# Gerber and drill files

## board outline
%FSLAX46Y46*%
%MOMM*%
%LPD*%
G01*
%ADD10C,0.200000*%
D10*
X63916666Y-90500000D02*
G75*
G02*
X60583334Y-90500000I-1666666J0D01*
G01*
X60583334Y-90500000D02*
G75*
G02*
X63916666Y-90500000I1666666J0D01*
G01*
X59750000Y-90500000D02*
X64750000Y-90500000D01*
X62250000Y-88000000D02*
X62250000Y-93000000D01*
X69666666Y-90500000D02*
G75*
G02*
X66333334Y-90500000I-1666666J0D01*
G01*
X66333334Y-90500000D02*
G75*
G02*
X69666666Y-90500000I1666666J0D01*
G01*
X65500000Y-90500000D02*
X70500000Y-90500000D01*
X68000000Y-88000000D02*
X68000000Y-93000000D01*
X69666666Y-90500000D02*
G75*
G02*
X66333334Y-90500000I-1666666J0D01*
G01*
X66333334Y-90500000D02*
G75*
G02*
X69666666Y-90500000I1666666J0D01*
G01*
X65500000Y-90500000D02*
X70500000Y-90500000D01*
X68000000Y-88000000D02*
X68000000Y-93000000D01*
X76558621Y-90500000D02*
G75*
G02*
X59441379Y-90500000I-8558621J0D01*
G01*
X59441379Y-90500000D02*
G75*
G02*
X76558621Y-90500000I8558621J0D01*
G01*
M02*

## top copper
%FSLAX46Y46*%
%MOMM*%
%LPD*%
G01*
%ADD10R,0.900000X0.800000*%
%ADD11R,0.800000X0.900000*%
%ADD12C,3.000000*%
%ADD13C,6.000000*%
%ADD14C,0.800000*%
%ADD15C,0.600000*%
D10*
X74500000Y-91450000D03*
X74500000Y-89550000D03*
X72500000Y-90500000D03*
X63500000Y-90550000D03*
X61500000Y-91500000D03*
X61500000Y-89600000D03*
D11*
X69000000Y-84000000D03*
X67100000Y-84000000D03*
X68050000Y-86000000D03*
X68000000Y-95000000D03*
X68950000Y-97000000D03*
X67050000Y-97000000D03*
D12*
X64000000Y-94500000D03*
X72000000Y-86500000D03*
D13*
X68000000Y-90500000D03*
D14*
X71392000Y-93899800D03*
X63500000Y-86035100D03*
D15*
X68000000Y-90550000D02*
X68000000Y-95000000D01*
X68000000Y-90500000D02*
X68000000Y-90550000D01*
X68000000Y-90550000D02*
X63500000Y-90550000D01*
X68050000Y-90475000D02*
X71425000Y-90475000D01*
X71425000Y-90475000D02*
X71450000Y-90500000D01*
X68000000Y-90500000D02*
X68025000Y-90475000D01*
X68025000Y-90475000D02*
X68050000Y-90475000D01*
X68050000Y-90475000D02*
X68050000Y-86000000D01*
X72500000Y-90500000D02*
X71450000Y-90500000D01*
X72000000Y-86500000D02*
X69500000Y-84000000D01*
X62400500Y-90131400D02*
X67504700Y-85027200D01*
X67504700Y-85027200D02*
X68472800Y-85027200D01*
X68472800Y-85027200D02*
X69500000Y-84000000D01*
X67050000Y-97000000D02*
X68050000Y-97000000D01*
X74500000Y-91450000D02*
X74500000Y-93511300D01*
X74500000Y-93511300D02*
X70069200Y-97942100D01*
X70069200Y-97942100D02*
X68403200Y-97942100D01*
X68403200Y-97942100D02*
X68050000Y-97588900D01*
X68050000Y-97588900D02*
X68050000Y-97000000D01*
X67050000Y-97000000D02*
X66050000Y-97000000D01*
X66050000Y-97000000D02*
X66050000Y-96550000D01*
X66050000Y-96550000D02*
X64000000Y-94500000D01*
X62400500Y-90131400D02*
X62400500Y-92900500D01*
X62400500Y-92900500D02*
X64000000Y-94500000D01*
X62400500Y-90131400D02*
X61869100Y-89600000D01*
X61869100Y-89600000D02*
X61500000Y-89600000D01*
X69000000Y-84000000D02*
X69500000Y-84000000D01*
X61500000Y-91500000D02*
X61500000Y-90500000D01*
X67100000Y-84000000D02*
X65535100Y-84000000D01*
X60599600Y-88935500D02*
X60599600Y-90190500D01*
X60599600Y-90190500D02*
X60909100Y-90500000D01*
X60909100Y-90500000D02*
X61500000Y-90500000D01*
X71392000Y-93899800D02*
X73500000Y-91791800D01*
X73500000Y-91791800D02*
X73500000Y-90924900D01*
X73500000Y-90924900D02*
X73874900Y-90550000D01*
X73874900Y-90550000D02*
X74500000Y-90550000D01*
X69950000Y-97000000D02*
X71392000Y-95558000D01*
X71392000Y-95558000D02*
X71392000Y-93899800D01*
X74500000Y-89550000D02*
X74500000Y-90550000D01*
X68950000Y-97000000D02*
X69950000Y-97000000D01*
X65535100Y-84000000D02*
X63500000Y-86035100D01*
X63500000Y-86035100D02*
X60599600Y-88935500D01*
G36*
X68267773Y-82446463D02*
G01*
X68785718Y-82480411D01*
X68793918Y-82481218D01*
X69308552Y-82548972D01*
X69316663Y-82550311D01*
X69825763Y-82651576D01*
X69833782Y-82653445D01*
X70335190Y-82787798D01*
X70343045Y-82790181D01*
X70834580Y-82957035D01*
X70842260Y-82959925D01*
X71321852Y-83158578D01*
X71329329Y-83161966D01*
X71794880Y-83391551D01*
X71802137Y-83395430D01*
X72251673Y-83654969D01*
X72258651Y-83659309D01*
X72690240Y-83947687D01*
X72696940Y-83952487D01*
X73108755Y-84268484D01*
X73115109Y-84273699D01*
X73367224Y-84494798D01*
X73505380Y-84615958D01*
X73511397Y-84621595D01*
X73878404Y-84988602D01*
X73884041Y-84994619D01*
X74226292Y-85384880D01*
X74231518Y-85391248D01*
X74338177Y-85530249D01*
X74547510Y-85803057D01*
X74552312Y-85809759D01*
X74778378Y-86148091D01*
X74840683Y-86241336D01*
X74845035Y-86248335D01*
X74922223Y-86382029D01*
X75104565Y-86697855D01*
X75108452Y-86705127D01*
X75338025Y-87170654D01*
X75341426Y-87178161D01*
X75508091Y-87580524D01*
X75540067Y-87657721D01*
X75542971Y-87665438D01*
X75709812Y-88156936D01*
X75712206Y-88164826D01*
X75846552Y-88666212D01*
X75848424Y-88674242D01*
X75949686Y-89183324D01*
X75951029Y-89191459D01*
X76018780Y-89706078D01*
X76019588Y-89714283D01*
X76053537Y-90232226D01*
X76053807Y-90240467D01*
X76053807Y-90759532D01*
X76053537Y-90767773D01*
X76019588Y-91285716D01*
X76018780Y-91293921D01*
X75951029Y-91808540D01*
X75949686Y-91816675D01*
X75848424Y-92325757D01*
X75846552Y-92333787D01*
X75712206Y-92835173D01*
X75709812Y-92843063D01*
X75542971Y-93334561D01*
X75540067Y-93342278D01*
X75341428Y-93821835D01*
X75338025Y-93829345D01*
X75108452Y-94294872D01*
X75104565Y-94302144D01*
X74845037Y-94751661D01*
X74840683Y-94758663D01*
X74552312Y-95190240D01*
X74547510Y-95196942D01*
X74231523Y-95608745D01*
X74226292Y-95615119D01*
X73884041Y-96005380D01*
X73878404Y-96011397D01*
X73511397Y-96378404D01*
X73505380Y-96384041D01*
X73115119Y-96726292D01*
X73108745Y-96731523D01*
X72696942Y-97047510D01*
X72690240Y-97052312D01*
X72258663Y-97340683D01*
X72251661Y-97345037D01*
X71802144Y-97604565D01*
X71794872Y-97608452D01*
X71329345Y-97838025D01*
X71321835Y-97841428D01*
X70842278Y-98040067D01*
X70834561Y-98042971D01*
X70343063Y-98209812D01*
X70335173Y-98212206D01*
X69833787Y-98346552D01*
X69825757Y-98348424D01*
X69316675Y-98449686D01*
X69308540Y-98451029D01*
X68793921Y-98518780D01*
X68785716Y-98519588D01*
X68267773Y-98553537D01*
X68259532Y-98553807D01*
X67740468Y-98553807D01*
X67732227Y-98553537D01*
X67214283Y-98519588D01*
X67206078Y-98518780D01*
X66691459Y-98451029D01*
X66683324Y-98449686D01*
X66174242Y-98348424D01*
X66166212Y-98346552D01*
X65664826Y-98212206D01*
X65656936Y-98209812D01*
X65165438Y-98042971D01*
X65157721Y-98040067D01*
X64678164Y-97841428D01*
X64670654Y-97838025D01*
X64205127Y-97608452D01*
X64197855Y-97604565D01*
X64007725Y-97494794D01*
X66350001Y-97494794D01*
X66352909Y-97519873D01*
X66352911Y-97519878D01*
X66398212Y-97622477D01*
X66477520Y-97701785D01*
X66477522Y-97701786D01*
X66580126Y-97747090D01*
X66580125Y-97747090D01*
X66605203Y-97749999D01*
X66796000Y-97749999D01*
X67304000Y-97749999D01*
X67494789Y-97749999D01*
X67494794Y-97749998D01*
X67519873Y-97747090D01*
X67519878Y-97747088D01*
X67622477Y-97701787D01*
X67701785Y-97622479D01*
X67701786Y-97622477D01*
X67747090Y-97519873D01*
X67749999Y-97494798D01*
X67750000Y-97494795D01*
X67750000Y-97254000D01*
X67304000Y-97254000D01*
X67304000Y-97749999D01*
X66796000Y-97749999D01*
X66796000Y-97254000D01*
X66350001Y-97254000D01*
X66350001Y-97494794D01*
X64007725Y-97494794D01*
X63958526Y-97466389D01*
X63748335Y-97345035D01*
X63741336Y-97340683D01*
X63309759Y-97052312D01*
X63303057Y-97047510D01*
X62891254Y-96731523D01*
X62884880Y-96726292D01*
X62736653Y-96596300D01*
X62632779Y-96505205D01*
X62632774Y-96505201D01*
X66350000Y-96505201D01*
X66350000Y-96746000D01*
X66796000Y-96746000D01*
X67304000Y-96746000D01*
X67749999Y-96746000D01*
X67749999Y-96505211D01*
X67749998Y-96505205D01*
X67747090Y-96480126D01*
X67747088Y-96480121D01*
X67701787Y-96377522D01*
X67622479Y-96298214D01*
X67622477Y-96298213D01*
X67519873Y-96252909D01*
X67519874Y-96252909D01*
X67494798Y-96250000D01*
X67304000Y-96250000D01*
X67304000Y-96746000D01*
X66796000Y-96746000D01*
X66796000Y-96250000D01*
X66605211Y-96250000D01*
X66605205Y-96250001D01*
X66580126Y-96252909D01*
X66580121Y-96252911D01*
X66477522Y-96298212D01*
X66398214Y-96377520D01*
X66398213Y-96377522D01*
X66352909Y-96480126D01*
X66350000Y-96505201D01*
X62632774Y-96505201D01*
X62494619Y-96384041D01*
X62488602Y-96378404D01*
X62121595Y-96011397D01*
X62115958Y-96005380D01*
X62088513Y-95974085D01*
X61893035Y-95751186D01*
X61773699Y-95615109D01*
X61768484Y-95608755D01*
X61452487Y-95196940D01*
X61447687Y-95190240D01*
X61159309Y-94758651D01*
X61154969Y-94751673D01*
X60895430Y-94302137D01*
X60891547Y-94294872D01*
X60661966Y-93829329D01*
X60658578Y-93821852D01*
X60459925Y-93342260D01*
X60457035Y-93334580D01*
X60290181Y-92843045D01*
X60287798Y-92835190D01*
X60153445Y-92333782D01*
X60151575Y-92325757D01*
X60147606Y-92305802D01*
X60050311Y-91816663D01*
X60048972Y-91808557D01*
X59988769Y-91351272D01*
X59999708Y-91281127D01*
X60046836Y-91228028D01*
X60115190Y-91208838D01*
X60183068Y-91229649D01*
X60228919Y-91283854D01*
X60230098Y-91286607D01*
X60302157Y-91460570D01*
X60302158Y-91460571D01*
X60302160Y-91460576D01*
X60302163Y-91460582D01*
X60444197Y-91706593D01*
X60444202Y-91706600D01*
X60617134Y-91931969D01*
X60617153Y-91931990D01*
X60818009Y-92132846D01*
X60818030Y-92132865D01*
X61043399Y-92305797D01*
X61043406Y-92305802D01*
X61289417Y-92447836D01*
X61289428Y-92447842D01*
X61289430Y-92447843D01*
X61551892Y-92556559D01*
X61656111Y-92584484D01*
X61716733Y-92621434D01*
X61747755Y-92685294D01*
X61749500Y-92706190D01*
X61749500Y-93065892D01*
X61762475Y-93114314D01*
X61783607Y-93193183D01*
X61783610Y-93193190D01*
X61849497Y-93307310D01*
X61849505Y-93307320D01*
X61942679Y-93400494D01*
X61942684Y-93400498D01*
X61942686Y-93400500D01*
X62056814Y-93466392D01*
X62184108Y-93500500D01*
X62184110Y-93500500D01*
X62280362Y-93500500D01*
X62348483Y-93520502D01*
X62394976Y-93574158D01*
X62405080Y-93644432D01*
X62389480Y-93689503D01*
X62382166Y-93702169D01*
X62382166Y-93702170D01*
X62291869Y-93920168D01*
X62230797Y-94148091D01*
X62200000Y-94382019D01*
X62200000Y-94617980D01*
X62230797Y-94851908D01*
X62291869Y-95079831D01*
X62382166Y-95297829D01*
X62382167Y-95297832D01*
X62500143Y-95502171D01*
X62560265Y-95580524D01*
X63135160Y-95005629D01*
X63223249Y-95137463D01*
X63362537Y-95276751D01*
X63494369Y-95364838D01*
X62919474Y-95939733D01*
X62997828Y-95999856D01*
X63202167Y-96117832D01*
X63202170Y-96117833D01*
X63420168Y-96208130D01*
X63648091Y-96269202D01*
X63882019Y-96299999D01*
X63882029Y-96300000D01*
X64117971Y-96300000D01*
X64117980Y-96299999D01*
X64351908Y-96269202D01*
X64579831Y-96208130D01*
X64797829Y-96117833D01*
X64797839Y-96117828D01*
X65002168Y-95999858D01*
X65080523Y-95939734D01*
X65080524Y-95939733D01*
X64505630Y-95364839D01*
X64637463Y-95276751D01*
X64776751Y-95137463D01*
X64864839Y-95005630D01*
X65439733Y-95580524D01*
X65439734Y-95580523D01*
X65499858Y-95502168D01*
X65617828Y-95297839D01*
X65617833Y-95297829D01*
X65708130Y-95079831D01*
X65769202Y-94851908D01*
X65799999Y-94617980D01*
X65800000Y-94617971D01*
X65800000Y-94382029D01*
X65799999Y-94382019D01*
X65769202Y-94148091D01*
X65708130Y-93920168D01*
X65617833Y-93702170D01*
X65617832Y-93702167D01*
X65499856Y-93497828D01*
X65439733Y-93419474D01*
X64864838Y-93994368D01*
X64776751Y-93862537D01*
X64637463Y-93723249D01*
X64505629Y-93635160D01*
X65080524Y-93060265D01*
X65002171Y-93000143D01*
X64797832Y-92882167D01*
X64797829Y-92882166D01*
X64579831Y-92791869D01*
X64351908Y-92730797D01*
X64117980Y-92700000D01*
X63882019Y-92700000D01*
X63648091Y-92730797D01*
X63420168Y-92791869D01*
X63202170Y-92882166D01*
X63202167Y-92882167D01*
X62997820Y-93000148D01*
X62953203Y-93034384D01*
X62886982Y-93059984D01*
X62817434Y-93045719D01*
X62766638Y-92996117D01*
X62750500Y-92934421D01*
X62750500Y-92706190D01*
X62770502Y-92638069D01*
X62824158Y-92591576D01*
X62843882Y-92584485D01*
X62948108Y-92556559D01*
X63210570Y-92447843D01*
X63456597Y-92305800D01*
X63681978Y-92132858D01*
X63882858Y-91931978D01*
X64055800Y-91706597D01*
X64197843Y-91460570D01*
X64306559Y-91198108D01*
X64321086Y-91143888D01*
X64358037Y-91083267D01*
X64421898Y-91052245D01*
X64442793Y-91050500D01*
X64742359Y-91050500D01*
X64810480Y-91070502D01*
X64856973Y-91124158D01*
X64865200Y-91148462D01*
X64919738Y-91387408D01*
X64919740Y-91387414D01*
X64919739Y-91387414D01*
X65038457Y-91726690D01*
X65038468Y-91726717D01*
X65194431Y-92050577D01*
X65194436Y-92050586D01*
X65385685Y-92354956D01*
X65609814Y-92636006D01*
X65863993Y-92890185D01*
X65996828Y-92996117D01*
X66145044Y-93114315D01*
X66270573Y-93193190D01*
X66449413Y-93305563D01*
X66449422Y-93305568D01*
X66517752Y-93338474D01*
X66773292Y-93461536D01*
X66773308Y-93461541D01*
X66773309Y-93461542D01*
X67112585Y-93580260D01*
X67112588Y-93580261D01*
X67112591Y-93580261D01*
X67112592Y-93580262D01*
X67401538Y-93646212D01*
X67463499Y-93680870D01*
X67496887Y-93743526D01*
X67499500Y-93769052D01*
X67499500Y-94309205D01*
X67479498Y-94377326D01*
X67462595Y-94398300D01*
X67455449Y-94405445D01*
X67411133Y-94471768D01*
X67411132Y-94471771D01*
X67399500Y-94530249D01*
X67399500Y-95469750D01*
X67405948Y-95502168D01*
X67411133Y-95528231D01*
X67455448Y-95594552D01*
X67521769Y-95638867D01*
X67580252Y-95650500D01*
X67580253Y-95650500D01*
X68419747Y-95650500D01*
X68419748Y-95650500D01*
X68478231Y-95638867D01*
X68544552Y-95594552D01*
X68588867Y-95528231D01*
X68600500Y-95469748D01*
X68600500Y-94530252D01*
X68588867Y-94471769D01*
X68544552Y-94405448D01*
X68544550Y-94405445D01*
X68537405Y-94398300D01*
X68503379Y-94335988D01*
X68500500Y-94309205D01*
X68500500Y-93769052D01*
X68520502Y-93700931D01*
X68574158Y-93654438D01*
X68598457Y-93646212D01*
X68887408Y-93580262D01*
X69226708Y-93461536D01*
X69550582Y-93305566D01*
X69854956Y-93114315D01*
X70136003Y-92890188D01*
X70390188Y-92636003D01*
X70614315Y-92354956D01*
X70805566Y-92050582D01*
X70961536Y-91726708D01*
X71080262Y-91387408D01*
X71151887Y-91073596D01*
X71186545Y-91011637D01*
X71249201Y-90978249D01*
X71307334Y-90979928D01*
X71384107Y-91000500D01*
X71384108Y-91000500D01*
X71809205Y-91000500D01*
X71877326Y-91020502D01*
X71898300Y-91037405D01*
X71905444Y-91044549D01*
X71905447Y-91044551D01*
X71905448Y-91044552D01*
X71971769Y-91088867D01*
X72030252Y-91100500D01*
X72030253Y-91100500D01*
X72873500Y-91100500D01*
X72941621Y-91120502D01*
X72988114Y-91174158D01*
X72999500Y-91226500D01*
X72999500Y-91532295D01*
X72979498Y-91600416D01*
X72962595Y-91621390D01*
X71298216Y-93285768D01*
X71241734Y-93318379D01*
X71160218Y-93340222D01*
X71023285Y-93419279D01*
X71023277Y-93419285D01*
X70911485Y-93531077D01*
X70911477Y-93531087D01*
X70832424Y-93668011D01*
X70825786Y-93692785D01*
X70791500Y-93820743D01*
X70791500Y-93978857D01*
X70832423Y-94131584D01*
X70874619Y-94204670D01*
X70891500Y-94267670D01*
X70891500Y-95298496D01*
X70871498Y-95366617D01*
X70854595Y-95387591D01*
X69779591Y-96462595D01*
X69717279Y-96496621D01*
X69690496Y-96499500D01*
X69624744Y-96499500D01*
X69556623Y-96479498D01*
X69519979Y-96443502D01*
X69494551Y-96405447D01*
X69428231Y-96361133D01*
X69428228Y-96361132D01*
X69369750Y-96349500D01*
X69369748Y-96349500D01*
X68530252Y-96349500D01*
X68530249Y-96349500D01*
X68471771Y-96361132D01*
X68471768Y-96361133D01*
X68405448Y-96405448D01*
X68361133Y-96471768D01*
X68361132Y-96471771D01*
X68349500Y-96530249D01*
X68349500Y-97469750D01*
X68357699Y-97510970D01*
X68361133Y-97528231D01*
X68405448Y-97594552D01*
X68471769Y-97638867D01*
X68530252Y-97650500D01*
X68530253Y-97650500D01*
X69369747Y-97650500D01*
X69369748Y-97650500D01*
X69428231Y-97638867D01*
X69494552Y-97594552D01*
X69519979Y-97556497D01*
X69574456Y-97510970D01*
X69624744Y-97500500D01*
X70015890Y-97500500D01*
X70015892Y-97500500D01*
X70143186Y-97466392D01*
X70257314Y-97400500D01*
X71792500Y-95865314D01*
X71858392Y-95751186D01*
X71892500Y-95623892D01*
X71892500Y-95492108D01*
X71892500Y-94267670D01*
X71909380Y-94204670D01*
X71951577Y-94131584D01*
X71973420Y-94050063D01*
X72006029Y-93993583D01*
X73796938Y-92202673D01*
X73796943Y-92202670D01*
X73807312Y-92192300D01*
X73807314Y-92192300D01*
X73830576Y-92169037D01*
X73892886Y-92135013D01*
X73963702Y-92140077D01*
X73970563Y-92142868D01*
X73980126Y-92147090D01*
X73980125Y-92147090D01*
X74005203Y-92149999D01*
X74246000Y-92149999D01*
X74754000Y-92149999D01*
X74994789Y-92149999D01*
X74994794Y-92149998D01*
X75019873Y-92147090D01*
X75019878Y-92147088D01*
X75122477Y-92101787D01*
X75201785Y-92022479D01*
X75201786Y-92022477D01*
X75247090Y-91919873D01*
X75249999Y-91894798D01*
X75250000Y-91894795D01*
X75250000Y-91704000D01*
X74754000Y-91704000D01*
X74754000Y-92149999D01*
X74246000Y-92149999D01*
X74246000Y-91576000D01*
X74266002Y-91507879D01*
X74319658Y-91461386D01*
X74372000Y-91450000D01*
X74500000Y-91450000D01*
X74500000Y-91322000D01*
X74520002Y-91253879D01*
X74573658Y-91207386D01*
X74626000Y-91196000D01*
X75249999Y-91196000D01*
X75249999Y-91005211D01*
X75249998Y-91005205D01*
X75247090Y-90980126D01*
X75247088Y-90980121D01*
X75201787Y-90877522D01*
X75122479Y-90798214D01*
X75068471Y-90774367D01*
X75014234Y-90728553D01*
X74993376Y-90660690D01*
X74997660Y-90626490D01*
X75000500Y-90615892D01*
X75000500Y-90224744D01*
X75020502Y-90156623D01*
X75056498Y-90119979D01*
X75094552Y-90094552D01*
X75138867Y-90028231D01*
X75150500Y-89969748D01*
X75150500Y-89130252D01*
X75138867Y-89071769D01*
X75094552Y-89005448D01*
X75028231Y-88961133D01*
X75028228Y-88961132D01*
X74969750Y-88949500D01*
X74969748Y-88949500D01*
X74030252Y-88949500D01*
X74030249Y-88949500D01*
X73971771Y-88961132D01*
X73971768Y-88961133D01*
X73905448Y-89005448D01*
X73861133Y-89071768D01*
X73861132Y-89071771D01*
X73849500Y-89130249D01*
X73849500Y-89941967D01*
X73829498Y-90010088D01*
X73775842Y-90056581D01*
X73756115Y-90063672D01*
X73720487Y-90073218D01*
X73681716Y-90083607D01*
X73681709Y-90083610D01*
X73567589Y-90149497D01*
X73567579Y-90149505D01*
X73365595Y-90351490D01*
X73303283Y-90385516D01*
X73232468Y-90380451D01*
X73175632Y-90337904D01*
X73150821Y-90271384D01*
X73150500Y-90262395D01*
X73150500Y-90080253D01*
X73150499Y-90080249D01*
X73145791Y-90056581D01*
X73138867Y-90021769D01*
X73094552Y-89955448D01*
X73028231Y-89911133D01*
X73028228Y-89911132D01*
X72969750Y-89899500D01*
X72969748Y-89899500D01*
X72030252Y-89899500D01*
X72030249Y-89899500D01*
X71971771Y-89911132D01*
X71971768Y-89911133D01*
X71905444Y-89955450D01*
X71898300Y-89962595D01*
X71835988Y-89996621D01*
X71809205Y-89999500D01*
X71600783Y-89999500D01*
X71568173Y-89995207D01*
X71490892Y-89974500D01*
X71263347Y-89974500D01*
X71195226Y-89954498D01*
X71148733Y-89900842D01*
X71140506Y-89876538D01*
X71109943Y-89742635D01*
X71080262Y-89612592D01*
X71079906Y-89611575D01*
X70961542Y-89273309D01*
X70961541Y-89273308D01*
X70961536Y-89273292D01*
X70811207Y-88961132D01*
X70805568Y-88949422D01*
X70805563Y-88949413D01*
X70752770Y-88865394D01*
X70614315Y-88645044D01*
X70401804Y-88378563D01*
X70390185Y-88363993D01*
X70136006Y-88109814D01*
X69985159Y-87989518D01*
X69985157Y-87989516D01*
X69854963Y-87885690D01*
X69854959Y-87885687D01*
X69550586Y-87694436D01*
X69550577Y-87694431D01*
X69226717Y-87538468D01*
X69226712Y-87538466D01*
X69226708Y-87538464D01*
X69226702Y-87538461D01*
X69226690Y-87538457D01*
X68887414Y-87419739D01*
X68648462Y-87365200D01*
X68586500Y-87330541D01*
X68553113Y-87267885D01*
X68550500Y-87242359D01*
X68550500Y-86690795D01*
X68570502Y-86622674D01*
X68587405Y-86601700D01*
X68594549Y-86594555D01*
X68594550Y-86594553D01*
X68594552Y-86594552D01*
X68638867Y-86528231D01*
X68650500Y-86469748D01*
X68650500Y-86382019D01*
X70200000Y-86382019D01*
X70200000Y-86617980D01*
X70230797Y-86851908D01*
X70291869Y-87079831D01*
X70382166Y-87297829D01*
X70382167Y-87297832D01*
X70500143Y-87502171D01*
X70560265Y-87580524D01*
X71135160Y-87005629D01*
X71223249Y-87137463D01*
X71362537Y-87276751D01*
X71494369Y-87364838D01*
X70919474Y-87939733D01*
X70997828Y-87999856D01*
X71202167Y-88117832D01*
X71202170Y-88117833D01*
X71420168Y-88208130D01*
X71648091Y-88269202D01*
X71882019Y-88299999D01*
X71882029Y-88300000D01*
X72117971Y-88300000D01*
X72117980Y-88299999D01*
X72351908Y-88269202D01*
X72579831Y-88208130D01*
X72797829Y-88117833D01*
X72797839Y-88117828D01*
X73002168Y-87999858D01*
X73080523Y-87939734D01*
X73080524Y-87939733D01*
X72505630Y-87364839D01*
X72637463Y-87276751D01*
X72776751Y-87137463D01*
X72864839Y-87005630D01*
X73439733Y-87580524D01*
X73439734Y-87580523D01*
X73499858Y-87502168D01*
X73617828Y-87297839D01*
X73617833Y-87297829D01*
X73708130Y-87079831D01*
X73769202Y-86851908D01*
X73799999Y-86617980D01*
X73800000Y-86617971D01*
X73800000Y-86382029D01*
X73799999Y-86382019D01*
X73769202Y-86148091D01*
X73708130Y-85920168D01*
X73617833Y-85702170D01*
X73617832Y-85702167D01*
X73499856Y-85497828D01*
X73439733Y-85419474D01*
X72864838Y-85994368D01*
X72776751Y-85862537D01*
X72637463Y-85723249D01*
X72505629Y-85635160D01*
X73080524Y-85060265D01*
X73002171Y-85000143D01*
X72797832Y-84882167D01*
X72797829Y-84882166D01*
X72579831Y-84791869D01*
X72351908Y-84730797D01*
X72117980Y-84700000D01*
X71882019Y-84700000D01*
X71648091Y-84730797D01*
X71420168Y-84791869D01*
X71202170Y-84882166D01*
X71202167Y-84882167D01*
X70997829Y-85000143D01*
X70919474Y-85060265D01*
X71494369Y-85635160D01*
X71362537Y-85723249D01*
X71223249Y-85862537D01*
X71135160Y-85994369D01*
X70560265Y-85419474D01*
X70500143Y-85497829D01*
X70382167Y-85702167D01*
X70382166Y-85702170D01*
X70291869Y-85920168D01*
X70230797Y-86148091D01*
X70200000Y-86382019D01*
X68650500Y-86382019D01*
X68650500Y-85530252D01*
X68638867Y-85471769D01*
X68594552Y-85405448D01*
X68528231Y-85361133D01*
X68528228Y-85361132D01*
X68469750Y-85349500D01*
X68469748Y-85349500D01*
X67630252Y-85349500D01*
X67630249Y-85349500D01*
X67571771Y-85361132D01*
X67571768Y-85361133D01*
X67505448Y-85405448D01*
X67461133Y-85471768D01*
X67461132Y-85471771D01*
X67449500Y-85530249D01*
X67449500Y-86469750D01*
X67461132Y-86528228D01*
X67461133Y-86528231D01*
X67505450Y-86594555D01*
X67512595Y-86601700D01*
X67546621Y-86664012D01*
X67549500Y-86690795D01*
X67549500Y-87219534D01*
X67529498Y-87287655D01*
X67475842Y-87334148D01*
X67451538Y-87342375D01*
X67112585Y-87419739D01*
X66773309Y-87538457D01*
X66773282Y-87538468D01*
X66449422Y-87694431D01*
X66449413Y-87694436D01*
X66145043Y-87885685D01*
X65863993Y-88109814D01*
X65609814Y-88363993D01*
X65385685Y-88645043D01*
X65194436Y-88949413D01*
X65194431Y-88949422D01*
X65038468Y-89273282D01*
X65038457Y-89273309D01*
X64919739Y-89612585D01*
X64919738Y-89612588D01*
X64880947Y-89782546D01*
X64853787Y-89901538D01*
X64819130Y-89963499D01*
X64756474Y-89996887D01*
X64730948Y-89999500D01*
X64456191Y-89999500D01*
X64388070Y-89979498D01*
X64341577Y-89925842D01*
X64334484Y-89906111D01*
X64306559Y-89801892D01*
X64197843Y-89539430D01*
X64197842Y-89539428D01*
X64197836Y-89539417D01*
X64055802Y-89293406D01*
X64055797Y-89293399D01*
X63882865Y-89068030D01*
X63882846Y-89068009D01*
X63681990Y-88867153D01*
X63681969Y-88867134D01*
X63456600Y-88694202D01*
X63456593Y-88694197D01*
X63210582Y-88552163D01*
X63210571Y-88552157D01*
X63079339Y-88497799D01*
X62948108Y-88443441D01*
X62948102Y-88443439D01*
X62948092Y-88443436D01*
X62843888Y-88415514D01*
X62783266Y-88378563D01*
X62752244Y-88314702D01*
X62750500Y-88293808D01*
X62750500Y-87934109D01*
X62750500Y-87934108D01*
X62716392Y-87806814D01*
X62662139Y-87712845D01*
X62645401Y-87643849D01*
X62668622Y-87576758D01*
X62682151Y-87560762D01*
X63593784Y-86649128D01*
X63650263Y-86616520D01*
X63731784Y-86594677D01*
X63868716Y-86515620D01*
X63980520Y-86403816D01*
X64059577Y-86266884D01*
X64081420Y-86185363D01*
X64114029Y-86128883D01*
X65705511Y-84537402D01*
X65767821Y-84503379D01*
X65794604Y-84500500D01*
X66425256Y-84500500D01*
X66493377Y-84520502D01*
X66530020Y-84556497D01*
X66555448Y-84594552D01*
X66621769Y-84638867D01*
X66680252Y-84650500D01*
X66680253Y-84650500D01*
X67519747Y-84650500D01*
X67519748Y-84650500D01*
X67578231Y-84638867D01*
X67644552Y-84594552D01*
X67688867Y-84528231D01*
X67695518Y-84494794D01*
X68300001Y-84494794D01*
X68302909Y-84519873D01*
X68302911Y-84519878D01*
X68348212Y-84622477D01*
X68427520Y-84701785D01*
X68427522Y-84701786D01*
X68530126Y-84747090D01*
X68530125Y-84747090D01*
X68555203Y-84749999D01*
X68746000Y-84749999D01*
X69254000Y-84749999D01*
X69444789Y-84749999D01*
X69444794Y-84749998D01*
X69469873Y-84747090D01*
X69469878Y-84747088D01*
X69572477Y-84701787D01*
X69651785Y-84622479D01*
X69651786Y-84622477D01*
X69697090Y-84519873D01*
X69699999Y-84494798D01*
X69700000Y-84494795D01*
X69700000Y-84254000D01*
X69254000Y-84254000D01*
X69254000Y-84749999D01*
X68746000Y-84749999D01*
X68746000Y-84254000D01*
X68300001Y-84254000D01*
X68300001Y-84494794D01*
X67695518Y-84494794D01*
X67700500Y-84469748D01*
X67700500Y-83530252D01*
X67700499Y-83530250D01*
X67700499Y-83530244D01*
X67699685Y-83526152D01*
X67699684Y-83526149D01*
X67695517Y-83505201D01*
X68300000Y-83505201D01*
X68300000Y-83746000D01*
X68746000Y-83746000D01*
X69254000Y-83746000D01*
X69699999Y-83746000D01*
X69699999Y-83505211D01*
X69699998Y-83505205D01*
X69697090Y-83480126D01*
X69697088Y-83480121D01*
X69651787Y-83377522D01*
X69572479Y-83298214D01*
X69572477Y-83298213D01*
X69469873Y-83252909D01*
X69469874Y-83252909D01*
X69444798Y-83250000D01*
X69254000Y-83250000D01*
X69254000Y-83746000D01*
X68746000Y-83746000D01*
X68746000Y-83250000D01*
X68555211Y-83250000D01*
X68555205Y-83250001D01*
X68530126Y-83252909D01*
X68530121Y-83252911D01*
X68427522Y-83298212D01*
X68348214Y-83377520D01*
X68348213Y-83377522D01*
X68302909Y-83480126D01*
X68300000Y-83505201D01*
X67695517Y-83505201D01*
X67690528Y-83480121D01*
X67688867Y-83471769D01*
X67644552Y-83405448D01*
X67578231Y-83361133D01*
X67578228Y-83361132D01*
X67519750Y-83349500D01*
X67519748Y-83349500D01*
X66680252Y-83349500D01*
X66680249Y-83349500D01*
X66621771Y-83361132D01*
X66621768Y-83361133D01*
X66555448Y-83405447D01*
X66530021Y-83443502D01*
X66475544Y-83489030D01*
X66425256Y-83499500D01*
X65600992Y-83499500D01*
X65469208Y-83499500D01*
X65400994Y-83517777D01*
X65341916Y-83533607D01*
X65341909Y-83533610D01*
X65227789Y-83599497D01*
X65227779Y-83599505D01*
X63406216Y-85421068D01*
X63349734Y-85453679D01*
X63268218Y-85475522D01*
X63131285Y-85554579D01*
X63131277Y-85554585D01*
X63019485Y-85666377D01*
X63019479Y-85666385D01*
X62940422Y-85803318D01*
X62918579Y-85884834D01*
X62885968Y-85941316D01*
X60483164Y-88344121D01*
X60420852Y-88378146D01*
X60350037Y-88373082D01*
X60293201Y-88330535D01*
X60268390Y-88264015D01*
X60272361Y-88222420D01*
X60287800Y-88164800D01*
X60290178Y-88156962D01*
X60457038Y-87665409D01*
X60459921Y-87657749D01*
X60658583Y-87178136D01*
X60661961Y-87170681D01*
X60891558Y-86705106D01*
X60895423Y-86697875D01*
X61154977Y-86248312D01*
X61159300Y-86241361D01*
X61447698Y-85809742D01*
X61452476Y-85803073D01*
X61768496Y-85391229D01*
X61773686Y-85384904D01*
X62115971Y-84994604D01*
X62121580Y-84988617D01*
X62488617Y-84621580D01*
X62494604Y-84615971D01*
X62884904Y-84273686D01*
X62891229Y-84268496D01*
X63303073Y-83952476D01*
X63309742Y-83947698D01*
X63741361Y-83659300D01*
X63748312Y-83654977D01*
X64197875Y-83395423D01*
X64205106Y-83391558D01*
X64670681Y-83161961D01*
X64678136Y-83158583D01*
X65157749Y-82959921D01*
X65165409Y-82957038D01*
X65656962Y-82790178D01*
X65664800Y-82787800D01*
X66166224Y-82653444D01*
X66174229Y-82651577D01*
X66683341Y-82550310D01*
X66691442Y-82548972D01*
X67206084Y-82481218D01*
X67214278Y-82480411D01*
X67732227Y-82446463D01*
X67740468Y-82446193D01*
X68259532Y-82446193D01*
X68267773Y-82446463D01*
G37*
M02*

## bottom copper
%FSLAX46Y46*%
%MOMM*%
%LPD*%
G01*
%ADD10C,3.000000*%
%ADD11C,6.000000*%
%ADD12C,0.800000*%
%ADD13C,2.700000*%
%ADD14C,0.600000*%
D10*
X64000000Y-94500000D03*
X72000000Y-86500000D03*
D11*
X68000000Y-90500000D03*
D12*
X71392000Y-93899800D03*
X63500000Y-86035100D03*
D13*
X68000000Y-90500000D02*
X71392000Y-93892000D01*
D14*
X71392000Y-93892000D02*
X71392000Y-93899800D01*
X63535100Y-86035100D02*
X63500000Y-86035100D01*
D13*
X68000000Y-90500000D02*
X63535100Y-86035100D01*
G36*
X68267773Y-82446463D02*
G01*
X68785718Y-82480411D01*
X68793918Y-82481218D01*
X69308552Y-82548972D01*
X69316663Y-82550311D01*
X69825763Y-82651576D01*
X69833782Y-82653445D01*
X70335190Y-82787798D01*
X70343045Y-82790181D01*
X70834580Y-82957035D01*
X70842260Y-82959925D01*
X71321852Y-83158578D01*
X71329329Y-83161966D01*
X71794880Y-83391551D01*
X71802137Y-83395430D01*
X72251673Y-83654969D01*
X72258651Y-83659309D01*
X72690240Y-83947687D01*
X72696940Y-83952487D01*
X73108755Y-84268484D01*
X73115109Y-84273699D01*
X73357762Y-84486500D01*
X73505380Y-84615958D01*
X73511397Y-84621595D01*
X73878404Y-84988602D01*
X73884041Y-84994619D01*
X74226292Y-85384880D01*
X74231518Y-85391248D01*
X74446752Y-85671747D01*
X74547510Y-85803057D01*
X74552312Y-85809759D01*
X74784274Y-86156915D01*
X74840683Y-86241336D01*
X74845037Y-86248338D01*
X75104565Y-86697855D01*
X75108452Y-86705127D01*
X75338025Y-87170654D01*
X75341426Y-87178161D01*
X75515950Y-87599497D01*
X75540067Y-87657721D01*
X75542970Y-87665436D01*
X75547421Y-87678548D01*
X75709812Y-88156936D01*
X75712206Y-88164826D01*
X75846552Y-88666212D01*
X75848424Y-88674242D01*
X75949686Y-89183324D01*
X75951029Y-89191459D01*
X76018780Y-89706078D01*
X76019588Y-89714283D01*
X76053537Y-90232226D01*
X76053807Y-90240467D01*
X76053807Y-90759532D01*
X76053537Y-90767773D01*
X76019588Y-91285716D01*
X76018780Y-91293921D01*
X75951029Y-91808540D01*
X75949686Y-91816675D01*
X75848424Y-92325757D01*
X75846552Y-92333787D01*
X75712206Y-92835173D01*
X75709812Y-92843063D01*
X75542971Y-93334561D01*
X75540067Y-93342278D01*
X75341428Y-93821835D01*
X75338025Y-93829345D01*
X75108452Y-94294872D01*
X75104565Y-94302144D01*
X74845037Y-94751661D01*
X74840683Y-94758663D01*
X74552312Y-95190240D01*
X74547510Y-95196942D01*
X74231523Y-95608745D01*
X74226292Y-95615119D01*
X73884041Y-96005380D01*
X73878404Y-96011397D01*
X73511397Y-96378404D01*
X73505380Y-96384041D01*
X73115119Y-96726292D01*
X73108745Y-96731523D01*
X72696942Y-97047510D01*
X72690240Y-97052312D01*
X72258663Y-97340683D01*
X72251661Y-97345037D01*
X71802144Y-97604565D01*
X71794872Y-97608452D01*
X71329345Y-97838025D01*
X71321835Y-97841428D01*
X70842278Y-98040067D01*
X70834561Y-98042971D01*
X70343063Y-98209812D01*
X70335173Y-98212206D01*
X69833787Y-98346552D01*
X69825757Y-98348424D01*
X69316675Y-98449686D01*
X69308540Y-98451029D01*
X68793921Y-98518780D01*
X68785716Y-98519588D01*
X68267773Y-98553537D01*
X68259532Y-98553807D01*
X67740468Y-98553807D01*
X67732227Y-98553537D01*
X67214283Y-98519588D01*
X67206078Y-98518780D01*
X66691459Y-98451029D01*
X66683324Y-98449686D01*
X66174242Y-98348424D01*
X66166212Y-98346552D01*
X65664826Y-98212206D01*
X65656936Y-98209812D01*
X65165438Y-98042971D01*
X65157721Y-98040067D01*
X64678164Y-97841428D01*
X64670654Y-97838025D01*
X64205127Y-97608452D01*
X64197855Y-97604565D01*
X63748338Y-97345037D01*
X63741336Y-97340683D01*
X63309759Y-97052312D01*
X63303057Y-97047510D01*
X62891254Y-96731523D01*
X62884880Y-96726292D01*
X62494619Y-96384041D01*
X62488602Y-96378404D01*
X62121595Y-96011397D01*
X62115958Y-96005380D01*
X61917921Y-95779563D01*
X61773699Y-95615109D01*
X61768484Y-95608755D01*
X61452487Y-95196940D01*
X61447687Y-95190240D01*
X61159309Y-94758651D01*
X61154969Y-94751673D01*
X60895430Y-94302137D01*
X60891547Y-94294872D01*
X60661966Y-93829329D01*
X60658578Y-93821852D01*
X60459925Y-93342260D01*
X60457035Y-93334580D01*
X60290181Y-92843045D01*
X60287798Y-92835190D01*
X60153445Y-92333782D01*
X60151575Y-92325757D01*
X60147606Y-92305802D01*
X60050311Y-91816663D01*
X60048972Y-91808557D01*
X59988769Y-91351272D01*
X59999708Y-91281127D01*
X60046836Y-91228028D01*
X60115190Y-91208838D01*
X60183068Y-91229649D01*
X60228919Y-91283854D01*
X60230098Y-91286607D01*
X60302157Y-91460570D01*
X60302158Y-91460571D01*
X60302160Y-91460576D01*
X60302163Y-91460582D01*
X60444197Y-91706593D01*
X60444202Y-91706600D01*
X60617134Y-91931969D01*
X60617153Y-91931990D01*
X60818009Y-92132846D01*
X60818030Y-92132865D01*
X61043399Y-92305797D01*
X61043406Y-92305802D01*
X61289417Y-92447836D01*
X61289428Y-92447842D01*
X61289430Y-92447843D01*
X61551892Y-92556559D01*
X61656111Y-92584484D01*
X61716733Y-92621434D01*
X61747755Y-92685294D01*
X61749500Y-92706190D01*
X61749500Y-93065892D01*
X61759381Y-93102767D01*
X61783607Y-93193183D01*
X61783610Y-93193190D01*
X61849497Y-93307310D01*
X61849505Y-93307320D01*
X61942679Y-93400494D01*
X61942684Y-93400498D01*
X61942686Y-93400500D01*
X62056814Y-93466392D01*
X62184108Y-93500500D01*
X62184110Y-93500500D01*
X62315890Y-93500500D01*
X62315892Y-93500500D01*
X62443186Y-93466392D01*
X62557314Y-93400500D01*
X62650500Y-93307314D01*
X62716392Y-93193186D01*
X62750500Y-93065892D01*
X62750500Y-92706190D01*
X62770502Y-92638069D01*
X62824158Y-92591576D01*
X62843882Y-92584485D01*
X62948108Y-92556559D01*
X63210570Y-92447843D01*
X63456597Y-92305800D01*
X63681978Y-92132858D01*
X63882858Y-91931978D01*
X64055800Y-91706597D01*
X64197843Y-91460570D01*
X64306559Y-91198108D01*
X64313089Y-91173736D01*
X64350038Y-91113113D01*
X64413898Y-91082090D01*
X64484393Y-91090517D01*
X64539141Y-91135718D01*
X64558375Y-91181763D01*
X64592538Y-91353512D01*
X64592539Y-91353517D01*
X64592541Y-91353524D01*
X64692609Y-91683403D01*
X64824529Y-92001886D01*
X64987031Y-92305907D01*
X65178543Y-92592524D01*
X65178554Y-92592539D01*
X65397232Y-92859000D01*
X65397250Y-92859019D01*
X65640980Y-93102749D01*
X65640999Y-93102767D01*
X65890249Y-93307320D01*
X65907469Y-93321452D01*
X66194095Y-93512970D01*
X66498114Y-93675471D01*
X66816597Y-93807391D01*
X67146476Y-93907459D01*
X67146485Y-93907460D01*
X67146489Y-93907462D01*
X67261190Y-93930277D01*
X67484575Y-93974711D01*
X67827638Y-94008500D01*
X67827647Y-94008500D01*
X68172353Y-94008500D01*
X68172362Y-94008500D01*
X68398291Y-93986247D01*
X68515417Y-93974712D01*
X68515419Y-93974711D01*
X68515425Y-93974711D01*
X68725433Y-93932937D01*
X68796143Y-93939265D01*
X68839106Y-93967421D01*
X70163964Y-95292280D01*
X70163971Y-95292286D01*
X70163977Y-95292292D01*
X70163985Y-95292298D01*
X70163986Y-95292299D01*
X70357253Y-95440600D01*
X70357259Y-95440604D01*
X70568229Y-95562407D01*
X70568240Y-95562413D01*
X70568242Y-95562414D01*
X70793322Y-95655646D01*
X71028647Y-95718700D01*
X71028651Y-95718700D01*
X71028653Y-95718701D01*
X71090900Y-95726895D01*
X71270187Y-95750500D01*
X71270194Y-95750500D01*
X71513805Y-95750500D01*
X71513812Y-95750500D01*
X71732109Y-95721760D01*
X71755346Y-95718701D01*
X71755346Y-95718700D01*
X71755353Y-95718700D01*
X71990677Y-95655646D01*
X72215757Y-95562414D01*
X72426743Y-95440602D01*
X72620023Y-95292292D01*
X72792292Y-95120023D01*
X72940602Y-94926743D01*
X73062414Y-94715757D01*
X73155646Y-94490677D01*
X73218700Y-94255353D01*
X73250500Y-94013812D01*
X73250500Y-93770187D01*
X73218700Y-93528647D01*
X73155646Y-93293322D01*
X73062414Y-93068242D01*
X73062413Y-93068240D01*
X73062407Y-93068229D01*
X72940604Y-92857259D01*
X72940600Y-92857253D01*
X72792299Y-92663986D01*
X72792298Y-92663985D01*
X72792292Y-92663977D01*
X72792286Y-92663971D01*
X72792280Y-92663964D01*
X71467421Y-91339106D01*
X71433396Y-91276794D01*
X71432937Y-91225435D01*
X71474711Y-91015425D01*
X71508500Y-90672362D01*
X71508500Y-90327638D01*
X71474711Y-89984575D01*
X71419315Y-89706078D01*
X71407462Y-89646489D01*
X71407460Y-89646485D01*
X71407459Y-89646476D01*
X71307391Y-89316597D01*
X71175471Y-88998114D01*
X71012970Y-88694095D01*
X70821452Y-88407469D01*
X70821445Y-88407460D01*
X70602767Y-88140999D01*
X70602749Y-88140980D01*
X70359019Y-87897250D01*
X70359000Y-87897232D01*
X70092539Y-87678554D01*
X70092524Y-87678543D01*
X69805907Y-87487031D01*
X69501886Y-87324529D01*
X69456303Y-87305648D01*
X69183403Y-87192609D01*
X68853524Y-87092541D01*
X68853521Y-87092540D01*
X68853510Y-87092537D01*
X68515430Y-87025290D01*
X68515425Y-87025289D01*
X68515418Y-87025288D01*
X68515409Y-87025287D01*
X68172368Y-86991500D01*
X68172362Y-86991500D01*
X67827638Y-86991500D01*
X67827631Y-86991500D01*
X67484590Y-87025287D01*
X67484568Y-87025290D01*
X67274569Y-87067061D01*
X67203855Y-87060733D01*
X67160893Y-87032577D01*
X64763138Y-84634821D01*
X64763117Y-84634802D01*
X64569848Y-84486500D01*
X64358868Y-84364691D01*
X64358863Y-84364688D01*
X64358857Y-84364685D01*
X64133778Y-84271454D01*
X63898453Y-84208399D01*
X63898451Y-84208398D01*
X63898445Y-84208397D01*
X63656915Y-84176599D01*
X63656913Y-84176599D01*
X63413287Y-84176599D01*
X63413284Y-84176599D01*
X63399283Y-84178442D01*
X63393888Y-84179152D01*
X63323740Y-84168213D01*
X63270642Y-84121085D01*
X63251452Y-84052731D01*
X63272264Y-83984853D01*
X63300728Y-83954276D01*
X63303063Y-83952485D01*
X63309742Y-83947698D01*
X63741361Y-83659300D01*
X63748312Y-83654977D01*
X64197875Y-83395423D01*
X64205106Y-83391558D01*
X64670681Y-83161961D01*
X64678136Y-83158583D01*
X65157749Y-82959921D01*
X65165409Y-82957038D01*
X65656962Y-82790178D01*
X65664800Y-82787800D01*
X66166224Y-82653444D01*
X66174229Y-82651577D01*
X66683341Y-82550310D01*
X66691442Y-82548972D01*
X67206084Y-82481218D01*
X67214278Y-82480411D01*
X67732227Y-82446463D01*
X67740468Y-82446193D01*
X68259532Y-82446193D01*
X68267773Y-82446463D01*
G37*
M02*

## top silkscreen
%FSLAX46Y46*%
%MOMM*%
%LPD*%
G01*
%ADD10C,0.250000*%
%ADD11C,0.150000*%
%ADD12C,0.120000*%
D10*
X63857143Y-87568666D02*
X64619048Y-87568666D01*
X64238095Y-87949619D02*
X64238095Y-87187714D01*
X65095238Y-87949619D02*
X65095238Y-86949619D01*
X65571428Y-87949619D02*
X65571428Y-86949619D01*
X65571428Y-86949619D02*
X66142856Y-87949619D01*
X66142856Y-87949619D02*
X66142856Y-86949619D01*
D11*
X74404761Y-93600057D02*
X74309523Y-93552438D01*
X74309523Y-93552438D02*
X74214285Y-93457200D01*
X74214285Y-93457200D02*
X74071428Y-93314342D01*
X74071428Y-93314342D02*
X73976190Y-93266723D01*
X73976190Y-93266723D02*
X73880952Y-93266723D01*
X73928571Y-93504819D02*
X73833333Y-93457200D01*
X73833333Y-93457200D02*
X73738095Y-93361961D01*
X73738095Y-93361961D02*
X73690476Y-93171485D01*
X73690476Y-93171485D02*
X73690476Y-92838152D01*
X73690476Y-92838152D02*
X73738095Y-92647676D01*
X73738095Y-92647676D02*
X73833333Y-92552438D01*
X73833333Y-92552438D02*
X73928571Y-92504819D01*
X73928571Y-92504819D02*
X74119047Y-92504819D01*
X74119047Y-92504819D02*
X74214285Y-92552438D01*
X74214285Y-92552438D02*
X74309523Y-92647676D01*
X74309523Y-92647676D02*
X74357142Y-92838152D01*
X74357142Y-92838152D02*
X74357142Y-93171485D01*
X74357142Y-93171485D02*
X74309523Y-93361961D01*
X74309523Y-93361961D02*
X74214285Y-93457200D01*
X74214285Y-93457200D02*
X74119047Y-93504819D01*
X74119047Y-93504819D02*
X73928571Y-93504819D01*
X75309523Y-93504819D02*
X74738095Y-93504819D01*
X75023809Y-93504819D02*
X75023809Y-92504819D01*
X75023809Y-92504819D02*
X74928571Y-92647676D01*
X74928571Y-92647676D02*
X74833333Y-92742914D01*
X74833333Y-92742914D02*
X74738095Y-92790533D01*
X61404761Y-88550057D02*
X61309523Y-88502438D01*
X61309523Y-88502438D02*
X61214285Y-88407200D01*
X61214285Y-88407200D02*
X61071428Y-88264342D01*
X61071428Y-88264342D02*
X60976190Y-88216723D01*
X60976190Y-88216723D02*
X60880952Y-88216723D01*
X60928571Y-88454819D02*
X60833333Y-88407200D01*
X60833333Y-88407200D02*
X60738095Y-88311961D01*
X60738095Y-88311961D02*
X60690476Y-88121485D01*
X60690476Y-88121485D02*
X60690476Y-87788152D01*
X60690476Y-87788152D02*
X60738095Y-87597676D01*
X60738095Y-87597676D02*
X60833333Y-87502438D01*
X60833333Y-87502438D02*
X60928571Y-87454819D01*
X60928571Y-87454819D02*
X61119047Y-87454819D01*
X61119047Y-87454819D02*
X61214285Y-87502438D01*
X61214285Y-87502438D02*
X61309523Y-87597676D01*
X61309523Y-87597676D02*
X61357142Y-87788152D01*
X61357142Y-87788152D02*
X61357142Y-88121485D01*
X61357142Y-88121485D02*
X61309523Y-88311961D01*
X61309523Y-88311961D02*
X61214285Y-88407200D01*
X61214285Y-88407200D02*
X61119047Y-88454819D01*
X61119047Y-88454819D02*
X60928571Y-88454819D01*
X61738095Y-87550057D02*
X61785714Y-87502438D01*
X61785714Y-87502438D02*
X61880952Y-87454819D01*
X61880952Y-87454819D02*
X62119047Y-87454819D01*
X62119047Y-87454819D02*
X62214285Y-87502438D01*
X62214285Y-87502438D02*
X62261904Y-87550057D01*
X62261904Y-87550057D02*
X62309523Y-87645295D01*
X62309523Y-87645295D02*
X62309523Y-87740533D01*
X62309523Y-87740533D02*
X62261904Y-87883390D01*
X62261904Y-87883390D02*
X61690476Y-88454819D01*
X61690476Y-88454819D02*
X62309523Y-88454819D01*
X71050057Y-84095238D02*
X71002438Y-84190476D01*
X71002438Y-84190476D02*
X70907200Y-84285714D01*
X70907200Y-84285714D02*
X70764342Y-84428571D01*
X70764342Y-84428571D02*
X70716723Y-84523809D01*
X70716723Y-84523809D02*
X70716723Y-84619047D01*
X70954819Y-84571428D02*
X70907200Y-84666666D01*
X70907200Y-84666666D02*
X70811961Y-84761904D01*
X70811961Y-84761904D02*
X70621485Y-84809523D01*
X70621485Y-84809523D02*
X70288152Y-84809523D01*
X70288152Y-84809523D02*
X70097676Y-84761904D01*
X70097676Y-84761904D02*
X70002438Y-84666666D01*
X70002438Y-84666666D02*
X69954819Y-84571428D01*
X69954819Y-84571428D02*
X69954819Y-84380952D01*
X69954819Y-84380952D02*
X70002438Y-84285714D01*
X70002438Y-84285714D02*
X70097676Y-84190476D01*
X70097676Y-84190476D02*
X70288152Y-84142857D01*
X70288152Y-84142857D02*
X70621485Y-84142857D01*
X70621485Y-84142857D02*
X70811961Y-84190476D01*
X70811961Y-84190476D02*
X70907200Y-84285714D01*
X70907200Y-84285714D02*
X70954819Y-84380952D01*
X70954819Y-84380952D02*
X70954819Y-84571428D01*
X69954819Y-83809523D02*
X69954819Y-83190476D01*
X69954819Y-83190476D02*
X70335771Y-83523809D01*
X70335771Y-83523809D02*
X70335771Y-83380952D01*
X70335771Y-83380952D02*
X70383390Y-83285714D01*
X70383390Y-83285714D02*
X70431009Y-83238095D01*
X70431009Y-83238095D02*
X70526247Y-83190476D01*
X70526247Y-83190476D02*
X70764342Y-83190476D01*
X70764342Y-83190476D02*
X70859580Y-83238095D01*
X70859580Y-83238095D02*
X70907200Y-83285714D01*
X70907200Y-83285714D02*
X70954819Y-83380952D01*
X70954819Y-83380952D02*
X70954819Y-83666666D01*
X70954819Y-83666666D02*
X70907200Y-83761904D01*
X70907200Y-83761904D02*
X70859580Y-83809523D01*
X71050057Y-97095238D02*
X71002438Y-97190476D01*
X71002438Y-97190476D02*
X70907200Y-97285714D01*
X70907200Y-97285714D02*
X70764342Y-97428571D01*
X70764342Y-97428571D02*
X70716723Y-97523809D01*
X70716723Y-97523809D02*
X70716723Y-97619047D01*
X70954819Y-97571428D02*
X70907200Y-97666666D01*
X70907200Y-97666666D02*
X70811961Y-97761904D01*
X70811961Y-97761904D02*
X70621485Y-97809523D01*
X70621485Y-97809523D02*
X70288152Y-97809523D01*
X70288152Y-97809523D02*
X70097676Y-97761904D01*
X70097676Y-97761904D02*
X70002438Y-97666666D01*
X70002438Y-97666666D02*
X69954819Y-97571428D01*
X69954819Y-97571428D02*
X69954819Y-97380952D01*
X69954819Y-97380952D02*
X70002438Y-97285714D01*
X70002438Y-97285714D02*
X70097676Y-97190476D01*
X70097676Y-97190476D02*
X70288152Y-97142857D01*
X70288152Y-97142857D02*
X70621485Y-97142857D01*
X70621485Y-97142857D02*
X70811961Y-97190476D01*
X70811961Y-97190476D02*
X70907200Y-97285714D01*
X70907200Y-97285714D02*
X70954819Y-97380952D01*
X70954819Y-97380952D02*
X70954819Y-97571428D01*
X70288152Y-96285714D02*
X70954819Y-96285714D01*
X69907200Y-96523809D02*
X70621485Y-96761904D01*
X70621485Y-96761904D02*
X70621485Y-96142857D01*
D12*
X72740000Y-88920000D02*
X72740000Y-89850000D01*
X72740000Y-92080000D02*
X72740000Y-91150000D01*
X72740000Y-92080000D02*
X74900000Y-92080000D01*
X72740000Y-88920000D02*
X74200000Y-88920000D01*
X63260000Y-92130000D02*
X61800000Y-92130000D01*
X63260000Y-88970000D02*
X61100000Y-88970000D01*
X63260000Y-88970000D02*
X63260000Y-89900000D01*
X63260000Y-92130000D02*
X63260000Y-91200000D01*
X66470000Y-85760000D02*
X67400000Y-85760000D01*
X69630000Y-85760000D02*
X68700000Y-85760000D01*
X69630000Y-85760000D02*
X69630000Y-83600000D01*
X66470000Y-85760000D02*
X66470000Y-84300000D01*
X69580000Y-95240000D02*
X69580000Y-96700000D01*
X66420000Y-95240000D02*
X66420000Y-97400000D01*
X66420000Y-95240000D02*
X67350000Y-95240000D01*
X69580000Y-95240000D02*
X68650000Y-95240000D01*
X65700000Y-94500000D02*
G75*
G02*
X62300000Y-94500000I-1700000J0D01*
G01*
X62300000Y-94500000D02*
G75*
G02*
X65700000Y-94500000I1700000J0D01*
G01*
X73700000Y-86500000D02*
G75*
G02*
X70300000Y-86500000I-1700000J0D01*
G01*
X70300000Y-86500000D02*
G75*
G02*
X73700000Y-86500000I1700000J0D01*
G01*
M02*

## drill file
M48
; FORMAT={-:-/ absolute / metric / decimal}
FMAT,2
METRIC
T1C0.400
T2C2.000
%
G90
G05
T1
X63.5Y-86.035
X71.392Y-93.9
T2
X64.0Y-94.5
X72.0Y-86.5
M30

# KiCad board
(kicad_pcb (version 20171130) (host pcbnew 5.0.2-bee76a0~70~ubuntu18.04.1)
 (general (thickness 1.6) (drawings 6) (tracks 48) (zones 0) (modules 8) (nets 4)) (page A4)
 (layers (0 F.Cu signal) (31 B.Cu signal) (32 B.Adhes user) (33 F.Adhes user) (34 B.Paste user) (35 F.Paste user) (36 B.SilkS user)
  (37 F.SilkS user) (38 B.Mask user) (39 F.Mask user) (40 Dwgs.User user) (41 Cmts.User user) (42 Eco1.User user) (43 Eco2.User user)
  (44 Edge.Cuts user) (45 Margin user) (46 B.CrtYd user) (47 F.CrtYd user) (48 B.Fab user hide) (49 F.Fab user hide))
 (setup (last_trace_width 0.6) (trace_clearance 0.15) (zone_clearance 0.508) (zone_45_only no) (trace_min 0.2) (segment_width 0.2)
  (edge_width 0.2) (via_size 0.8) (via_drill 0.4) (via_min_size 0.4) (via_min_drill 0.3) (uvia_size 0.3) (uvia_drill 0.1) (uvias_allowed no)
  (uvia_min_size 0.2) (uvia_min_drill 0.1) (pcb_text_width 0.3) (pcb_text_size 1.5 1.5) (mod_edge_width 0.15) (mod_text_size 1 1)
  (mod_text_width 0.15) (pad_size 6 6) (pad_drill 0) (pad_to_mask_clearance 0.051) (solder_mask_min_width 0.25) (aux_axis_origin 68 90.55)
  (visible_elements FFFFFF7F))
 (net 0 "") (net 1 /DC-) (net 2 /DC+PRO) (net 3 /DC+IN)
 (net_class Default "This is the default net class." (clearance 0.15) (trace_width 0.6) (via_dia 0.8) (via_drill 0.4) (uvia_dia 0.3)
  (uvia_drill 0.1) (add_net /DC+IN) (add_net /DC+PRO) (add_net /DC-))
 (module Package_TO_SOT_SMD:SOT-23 (layer F.Cu) (at 73.5 90.5 180)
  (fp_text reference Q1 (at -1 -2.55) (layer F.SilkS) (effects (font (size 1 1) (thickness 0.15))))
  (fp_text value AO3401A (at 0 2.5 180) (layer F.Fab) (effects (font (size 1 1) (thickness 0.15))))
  (fp_line (start 0.76 1.58) (end 0.76 0.65) (layer F.SilkS) (width 0.12))
  (fp_line (start 0.76 -1.58) (end 0.76 -0.65) (layer F.SilkS) (width 0.12))
  (fp_line (start 0.76 -1.58) (end -1.4 -1.58) (layer F.SilkS) (width 0.12))
  (fp_line (start 0.76 1.58) (end -0.7 1.58) (layer F.SilkS) (width 0.12))
  (pad 1 smd rect (at -1 -0.95 180) (size 0.9 0.8) (layers F.Cu F.Paste F.Mask) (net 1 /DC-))
  (pad 2 smd rect (at -1 0.95 180) (size 0.9 0.8) (layers F.Cu F.Paste F.Mask) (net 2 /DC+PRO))
  (pad 3 smd rect (at 1 0 180) (size 0.9 0.8) (layers F.Cu F.Paste F.Mask) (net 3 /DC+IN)))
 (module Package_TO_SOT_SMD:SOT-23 (layer F.Cu) (at 62.5 90.55)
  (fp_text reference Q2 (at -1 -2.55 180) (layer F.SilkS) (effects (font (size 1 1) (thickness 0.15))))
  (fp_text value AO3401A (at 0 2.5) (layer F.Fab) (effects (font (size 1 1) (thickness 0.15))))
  (fp_line (start 0.76 1.58) (end -0.7 1.58) (layer F.SilkS) (width 0.12))
  (fp_line (start 0.76 -1.58) (end -1.4 -1.58) (layer F.SilkS) (width 0.12))
  (fp_line (start 0.76 -1.58) (end 0.76 -0.65) (layer F.SilkS) (width 0.12))
  (fp_line (start 0.76 1.58) (end 0.76 0.65) (layer F.SilkS) (width 0.12))
  (pad 3 smd rect (at 1 0) (size 0.9 0.8) (layers F.Cu F.Paste F.Mask) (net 3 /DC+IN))
  (pad 2 smd rect (at -1 0.95) (size 0.9 0.8) (layers F.Cu F.Paste F.Mask) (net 2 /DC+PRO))
  (pad 1 smd rect (at -1 -0.95) (size 0.9 0.8) (layers F.Cu F.Paste F.Mask) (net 1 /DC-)))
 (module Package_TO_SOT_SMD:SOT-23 (layer F.Cu) (at 68.05 85 270)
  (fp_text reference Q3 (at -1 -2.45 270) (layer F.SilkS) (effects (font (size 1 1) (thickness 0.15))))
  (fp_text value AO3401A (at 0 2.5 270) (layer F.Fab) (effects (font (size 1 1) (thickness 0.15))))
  (fp_line (start 0.76 1.58) (end 0.76 0.65) (layer F.SilkS) (width 0.12))
  (fp_line (start 0.76 -1.58) (end 0.76 -0.65) (layer F.SilkS) (width 0.12))
  (fp_line (start 0.76 -1.58) (end -1.4 -1.58) (layer F.SilkS) (width 0.12))
  (fp_line (start 0.76 1.58) (end -0.7 1.58) (layer F.SilkS) (width 0.12))
  (pad 1 smd rect (at -1 -0.95 270) (size 0.9 0.8) (layers F.Cu F.Paste F.Mask) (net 1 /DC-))
  (pad 2 smd rect (at -1 0.95 270) (size 0.9 0.8) (layers F.Cu F.Paste F.Mask) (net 2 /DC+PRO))
  (pad 3 smd rect (at 1 0 270) (size 0.9 0.8) (layers F.Cu F.Paste F.Mask) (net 3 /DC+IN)))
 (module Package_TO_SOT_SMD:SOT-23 (layer F.Cu) (at 68 96 90)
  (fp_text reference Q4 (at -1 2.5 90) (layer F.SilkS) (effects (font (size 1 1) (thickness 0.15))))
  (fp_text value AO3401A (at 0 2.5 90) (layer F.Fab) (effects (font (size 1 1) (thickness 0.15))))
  (fp_line (start 0.76 1.58) (end -0.7 1.58) (layer F.SilkS) (width 0.12))
  (fp_line (start 0.76 -1.58) (end -1.4 -1.58) (layer F.SilkS) (width 0.12))
  (fp_line (start 0.76 -1.58) (end 0.76 -0.65) (layer F.SilkS) (width 0.12))
  (fp_line (start 0.76 1.58) (end 0.76 0.65) (layer F.SilkS) (width 0.12))
  (pad 3 smd rect (at 1 0 90) (size 0.9 0.8) (layers F.Cu F.Paste F.Mask) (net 3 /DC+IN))
  (pad 2 smd rect (at -1 0.95 90) (size 0.9 0.8) (layers F.Cu F.Paste F.Mask) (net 2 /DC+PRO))
  (pad 1 smd rect (at -1 -0.95 90) (size 0.9 0.8) (layers F.Cu F.Paste F.Mask) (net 1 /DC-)))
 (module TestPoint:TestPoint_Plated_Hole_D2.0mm (layer F.Cu) (at 64 94.5)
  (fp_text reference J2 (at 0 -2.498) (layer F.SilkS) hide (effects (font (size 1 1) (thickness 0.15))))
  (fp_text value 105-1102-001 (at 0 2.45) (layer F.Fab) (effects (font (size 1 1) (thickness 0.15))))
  (fp_circle (center 0 0) (end 0 -1.7) (layer F.SilkS) (width 0.12))
  (pad 1 thru_hole circle (at 0 0) (size 3 3) (drill 2) (layers *.Cu *.Mask) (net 1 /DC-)))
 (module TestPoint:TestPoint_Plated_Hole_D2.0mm (layer F.Cu) (at 72 86.5)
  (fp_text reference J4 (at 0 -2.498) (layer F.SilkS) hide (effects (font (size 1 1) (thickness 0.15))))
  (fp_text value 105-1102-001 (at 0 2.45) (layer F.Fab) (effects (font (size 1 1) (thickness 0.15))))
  (fp_circle (center 0 0) (end 0 -1.7) (layer F.SilkS) (width 0.12))
  (pad 1 thru_hole circle (at 0 0) (size 3 3) (drill 2) (layers *.Cu *.Mask) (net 1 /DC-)))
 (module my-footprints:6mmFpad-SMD (layer F.Cu) (at 68 90.5)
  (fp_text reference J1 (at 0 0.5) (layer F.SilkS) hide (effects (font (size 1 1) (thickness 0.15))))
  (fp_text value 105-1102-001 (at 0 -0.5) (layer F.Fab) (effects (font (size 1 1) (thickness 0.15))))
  (pad 1 smd circle (at 0 0) (size 6 6) (layers F.Cu F.Paste F.Mask) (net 3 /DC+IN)))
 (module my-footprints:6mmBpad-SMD (layer F.Cu) (at 68 90.5)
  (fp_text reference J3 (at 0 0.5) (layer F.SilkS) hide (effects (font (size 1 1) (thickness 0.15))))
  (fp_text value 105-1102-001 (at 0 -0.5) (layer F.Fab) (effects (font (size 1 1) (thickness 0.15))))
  (pad 1 smd circle (at 0 0) (size 6 6) (layers B.Cu B.Paste B.Mask) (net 2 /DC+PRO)))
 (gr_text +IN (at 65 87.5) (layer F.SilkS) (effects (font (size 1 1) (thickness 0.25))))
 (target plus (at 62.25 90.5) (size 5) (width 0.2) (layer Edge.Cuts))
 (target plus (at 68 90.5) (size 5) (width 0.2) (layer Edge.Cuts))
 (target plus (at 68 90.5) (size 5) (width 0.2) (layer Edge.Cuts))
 (gr_circle (center 68 90.5) (end 76.558621 90.5) (layer Edge.Cuts) (width 0.2))
 (segment (start 68 90.55) (end 68 95) (width 0.6) (layer F.Cu) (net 3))
 (segment (start 68 90.5) (end 68 90.55) (width 0.6) (layer F.Cu) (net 3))
 (segment (start 68 90.55) (end 63.5 90.55) (width 0.6) (layer F.Cu) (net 3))
 (segment (start 68.05 90.475) (end 71.425 90.475) (width 0.6) (layer F.Cu) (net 3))
 (segment (start 71.425 90.475) (end 71.45 90.5) (width 0.6) (layer F.Cu) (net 3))
 (segment (start 68 90.5) (end 68.025 90.475) (width 0.6) (layer F.Cu) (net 3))
 (segment (start 68.025 90.475) (end 68.05 90.475) (width 0.6) (layer F.Cu) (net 3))
 (segment (start 68.05 90.475) (end 68.05 86) (width 0.6) (layer F.Cu) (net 3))
 (segment (start 72.5 90.5) (end 71.45 90.5) (width 0.6) (layer F.Cu) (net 3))
 (segment (start 72 86.5) (end 69.5 84) (width 0.6) (layer F.Cu) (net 1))
 (segment (start 62.4005 90.1314) (end 67.5047 85.0272) (width 0.6) (layer F.Cu) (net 1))
 (segment (start 67.5047 85.0272) (end 68.4728 85.0272) (width 0.6) (layer F.Cu) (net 1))
 (segment (start 68.4728 85.0272) (end 69.5 84) (width 0.6) (layer F.Cu) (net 1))
 (segment (start 67.05 97) (end 68.05 97) (width 0.6) (layer F.Cu) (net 1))
 (segment (start 74.5 91.45) (end 74.5 93.5113) (width 0.6) (layer F.Cu) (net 1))
 (segment (start 74.5 93.5113) (end 70.0692 97.9421) (width 0.6) (layer F.Cu) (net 1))
 (segment (start 70.0692 97.9421) (end 68.4032 97.9421) (width 0.6) (layer F.Cu) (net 1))
 (segment (start 68.4032 97.9421) (end 68.05 97.5889) (width 0.6) (layer F.Cu) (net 1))
 (segment (start 68.05 97.5889) (end 68.05 97) (width 0.6) (layer F.Cu) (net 1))
 (segment (start 67.05 97) (end 66.05 97) (width 0.6) (layer F.Cu) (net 1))
 (segment (start 66.05 97) (end 66.05 96.55) (width 0.6) (layer F.Cu) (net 1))
 (segment (start 66.05 96.55) (end 64 94.5) (width 0.6) (layer F.Cu) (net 1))
 (segment (start 62.4005 90.1314) (end 62.4005 92.9005) (width 0.6) (layer F.Cu) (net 1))
 (segment (start 62.4005 92.9005) (end 64 94.5) (width 0.6) (layer F.Cu) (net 1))
 (segment (start 62.4005 90.1314) (end 61.8691 89.6) (width 0.6) (layer F.Cu) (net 1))
 (segment (start 61.8691 89.6) (end 61.5 89.6) (width 0.6) (layer F.Cu) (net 1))
 (segment (start 69 84) (end 69.5 84) (width 0.6) (layer F.Cu) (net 1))
 (segment (start 61.5 91.5) (end 61.5 90.5) (width 0.6) (layer F.Cu) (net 2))
 (segment (start 67.1 84) (end 65.5351 84) (width 0.6) (layer F.Cu) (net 2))
 (segment (start 60.5996 88.9355) (end 60.5996 90.1905) (width 0.6) (layer F.Cu) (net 2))
 (segment (start 60.5996 90.1905) (end 60.9091 90.5) (width 0.6) (layer F.Cu) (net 2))
 (segment (start 60.9091 90.5) (end 61.5 90.5) (width 0.6) (layer F.Cu) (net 2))
 (segment (start 71.392 93.8998) (end 73.5 91.7918) (width 0.6) (layer F.Cu) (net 2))
 (segment (start 73.5 91.7918) (end 73.5 90.9249) (width 0.6) (layer F.Cu) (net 2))
 (segment (start 73.5 90.9249) (end 73.8749 90.55) (width 0.6) (layer F.Cu) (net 2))
 (segment (start 73.8749 90.55) (end 74.5 90.55) (width 0.6) (layer F.Cu) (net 2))
 (segment (start 69.95 97) (end 71.392 95.558) (width 0.6) (layer F.Cu) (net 2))
 (segment (start 71.392 95.558) (end 71.392 93.8998) (width 0.6) (layer F.Cu) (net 2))
 (segment (start 68 90.5) (end 71.392 93.892) (width 2.7) (layer B.Cu) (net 2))
 (segment (start 71.392 93.892) (end 71.392 93.8998) (width 0.6) (layer B.Cu) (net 2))
 (segment (start 74.5 89.55) (end 74.5 90.55) (width 0.6) (layer F.Cu) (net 2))
 (segment (start 68.95 97) (end 69.95 97) (width 0.6) (layer F.Cu) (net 2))
 (via (at 71.392 93.8998) (size 0.8) (layers F.Cu B.Cu) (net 2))
 (segment (start 63.5351 86.0351) (end 63.5 86.0351) (width 0.6) (layer B.Cu) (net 2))
 (via (at 63.5 86.0351) (size 0.8) (drill 0.4) (layers F.Cu B.Cu) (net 2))
 (segment (start 68 90.5) (end 63.5351 86.0351) (width 2.7) (layer B.Cu) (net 2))
 (segment (start 65.5351 84) (end 63.5 86.0351) (width 0.6) (layer F.Cu) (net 2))
 (segment (start 63.5 86.0351) (end 60.5996 88.9355) (width 0.6) (layer F.Cu) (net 2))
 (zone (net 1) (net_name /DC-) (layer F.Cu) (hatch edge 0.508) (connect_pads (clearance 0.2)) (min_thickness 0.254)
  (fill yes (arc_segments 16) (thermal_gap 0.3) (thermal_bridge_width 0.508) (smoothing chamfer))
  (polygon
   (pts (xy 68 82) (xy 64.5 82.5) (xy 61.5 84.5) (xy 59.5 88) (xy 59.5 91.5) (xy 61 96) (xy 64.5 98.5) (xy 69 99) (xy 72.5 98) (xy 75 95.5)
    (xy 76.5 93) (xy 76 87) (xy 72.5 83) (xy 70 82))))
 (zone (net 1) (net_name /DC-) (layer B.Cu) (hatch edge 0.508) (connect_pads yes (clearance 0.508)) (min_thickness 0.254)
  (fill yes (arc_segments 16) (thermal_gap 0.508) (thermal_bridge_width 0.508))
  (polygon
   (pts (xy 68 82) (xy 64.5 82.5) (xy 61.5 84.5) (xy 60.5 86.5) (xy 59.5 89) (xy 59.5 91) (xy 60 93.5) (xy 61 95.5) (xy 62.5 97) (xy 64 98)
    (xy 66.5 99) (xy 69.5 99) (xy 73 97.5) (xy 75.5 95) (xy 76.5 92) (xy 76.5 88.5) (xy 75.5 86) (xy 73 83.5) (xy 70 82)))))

